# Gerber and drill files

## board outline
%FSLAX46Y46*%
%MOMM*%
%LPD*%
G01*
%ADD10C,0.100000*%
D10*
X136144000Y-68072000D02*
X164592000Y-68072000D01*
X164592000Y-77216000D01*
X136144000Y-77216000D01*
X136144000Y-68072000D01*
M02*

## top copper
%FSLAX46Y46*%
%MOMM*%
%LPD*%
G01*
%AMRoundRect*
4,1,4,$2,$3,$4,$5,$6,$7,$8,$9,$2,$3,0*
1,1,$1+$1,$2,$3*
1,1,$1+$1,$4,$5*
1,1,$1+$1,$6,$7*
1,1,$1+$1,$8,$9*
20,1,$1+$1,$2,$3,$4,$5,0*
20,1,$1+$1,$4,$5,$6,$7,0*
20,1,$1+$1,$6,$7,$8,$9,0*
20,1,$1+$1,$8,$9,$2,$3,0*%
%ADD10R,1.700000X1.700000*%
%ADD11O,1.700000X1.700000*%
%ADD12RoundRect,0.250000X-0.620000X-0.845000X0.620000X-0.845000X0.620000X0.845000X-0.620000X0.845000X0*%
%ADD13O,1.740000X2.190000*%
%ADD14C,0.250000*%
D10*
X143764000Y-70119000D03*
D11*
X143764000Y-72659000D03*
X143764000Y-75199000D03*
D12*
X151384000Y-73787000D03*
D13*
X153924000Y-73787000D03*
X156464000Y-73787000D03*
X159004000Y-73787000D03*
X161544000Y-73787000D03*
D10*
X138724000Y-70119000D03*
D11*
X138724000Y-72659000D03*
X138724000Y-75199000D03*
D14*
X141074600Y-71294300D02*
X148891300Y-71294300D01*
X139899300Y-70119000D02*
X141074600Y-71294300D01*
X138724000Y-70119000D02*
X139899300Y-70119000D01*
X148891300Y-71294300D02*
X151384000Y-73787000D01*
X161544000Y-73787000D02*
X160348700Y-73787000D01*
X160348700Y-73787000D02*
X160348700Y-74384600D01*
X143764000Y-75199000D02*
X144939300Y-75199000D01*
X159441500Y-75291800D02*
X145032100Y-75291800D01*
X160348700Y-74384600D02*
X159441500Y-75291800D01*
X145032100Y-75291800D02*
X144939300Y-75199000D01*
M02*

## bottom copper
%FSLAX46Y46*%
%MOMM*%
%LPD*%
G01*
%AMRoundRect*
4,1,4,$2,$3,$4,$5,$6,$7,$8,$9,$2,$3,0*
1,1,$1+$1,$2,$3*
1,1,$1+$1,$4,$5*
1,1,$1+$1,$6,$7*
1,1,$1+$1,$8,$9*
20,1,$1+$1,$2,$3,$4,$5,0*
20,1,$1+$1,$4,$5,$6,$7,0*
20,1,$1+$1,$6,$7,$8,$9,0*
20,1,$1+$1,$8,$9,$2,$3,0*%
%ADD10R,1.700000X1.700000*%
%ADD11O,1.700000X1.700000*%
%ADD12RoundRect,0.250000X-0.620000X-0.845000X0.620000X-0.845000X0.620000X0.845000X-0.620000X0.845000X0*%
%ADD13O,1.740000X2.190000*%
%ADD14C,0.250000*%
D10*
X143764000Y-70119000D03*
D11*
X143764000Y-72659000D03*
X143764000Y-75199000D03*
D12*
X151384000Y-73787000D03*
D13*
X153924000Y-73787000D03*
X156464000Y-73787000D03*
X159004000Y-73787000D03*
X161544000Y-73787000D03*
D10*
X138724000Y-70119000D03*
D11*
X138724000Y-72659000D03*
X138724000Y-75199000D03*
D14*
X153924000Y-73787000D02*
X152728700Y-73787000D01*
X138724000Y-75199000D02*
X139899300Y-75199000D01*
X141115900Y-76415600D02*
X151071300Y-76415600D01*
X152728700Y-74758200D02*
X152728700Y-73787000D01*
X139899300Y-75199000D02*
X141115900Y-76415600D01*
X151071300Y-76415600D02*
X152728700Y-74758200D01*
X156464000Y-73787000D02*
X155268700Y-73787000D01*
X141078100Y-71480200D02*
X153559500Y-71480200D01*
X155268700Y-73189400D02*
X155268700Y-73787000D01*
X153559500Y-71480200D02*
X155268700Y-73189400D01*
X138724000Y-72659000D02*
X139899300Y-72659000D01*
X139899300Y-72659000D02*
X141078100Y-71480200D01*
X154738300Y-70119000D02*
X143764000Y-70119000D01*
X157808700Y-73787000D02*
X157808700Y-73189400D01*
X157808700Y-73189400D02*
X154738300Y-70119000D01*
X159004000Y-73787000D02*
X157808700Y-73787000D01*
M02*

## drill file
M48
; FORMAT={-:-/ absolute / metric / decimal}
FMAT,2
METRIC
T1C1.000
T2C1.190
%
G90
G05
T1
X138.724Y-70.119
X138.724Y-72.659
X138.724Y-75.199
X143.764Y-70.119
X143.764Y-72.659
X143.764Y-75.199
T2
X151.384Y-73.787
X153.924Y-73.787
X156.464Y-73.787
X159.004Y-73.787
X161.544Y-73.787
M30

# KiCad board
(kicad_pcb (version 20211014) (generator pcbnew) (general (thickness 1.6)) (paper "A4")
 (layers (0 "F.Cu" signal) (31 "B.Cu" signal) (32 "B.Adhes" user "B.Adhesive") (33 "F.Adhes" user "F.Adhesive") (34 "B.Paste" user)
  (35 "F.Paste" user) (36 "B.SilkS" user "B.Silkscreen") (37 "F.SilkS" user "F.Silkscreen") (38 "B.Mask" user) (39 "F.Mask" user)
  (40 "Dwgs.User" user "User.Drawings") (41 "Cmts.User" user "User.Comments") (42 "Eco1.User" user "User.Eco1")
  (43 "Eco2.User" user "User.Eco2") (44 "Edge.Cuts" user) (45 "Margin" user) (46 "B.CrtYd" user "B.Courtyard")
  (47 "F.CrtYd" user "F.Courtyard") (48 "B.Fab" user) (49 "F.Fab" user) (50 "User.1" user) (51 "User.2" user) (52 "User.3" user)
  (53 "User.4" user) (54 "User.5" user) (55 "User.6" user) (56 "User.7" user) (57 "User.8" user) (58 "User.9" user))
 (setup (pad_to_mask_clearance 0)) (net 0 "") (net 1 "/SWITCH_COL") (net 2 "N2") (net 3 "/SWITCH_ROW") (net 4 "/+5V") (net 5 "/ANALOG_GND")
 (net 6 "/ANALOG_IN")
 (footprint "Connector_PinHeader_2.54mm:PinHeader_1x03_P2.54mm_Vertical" (layer "F.Cu") (at 143.764 70.119)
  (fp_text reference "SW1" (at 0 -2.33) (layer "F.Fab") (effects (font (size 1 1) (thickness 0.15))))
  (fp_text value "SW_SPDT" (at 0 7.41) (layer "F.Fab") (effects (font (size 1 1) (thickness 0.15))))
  (pad "1" thru_hole rect (at 0 0) (size 1.7 1.7) (drill 1) (layers *.Cu *.Mask) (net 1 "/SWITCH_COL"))
  (pad "2" thru_hole oval (at 0 2.54) (size 1.7 1.7) (drill 1) (layers *.Cu *.Mask) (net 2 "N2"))
  (pad "3" thru_hole oval (at 0 5.08) (size 1.7 1.7) (drill 1) (layers *.Cu *.Mask) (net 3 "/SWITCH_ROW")))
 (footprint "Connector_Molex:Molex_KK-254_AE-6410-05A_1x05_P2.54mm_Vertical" (layer "F.Cu") (at 151.384 73.787)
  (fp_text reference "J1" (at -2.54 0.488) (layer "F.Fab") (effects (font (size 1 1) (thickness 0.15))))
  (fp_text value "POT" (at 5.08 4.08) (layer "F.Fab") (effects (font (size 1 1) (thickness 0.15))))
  (pad "1" thru_hole roundrect (at 0 0) (size 1.74 2.19) (drill 1.19) (layers *.Cu *.Mask) (roundrect_rratio 0.1436781609) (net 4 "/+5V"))
  (pad "2" thru_hole oval (at 2.54 0) (size 1.74 2.19) (drill 1.19) (layers *.Cu *.Mask) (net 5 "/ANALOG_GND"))
  (pad "3" thru_hole oval (at 5.08 0) (size 1.74 2.19) (drill 1.19) (layers *.Cu *.Mask) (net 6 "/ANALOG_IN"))
  (pad "4" thru_hole oval (at 7.62 0) (size 1.74 2.19) (drill 1.19) (layers *.Cu *.Mask) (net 1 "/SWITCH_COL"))
  (pad "5" thru_hole oval (at 10.16 0) (size 1.74 2.19) (drill 1.19) (layers *.Cu *.Mask) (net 3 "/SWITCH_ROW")))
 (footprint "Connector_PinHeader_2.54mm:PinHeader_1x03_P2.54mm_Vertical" (layer "F.Cu") (at 138.724 70.119)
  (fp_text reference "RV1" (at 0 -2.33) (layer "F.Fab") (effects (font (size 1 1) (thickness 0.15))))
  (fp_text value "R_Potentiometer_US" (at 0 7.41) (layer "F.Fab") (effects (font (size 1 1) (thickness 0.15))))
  (pad "1" thru_hole rect (at 0 0) (size 1.7 1.7) (drill 1) (layers *.Cu *.Mask) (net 4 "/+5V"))
  (pad "2" thru_hole oval (at 0 2.54) (size 1.7 1.7) (drill 1) (layers *.Cu *.Mask) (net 6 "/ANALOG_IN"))
  (pad "3" thru_hole oval (at 0 5.08) (size 1.7 1.7) (drill 1) (layers *.Cu *.Mask) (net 5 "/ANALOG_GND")))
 (gr_rect (start 136.144 68.072) (end 164.592 77.216) (layer "Edge.Cuts") (width 0.1) (fill none))
 (segment (start 141.0746 71.2943) (end 148.8913 71.2943) (width 0.25) (layer "F.Cu") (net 4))
 (segment (start 139.8993 70.119) (end 141.0746 71.2943) (width 0.25) (layer "F.Cu") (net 4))
 (segment (start 138.724 70.119) (end 139.8993 70.119) (width 0.25) (layer "F.Cu") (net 4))
 (segment (start 148.8913 71.2943) (end 151.384 73.787) (width 0.25) (layer "F.Cu") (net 4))
 (segment (start 153.924 73.787) (end 152.7287 73.787) (width 0.25) (layer "B.Cu") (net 5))
 (segment (start 138.724 75.199) (end 139.8993 75.199) (width 0.25) (layer "B.Cu") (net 5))
 (segment (start 141.1159 76.4156) (end 151.0713 76.4156) (width 0.25) (layer "B.Cu") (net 5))
 (segment (start 152.7287 74.7582) (end 152.7287 73.787) (width 0.25) (layer "B.Cu") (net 5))
 (segment (start 139.8993 75.199) (end 141.1159 76.4156) (width 0.25) (layer "B.Cu") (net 5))
 (segment (start 151.0713 76.4156) (end 152.7287 74.7582) (width 0.25) (layer "B.Cu") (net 5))
 (segment (start 156.464 73.787) (end 155.2687 73.787) (width 0.25) (layer "B.Cu") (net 6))
 (segment (start 141.0781 71.4802) (end 153.5595 71.4802) (width 0.25) (layer "B.Cu") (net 6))
 (segment (start 155.2687 73.1894) (end 155.2687 73.787) (width 0.25) (layer "B.Cu") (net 6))
 (segment (start 153.5595 71.4802) (end 155.2687 73.1894) (width 0.25) (layer "B.Cu") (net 6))
 (segment (start 138.724 72.659) (end 139.8993 72.659) (width 0.25) (layer "B.Cu") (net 6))
 (segment (start 139.8993 72.659) (end 141.0781 71.4802) (width 0.25) (layer "B.Cu") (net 6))
 (segment (start 154.7383 70.119) (end 143.764 70.119) (width 0.25) (layer "B.Cu") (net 1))
 (segment (start 157.8087 73.787) (end 157.8087 73.1894) (width 0.25) (layer "B.Cu") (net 1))
 (segment (start 157.8087 73.1894) (end 154.7383 70.119) (width 0.25) (layer "B.Cu") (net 1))
 (segment (start 159.004 73.787) (end 157.8087 73.787) (width 0.25) (layer "B.Cu") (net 1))
 (segment (start 161.544 73.787) (end 160.3487 73.787) (width 0.25) (layer "F.Cu") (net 3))
 (segment (start 160.3487 73.787) (end 160.3487 74.3846) (width 0.25) (layer "F.Cu") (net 3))
 (segment (start 143.764 75.199) (end 144.9393 75.199) (width 0.25) (layer "F.Cu") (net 3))
 (segment (start 159.4415 75.2918) (end 145.0321 75.2918) (width 0.25) (layer "F.Cu") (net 3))
 (segment (start 160.3487 74.3846) (end 159.4415 75.2918) (width 0.25) (layer "F.Cu") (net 3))
 (segment (start 145.0321 75.2918) (end 144.9393 75.199) (width 0.25) (layer "F.Cu") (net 3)))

